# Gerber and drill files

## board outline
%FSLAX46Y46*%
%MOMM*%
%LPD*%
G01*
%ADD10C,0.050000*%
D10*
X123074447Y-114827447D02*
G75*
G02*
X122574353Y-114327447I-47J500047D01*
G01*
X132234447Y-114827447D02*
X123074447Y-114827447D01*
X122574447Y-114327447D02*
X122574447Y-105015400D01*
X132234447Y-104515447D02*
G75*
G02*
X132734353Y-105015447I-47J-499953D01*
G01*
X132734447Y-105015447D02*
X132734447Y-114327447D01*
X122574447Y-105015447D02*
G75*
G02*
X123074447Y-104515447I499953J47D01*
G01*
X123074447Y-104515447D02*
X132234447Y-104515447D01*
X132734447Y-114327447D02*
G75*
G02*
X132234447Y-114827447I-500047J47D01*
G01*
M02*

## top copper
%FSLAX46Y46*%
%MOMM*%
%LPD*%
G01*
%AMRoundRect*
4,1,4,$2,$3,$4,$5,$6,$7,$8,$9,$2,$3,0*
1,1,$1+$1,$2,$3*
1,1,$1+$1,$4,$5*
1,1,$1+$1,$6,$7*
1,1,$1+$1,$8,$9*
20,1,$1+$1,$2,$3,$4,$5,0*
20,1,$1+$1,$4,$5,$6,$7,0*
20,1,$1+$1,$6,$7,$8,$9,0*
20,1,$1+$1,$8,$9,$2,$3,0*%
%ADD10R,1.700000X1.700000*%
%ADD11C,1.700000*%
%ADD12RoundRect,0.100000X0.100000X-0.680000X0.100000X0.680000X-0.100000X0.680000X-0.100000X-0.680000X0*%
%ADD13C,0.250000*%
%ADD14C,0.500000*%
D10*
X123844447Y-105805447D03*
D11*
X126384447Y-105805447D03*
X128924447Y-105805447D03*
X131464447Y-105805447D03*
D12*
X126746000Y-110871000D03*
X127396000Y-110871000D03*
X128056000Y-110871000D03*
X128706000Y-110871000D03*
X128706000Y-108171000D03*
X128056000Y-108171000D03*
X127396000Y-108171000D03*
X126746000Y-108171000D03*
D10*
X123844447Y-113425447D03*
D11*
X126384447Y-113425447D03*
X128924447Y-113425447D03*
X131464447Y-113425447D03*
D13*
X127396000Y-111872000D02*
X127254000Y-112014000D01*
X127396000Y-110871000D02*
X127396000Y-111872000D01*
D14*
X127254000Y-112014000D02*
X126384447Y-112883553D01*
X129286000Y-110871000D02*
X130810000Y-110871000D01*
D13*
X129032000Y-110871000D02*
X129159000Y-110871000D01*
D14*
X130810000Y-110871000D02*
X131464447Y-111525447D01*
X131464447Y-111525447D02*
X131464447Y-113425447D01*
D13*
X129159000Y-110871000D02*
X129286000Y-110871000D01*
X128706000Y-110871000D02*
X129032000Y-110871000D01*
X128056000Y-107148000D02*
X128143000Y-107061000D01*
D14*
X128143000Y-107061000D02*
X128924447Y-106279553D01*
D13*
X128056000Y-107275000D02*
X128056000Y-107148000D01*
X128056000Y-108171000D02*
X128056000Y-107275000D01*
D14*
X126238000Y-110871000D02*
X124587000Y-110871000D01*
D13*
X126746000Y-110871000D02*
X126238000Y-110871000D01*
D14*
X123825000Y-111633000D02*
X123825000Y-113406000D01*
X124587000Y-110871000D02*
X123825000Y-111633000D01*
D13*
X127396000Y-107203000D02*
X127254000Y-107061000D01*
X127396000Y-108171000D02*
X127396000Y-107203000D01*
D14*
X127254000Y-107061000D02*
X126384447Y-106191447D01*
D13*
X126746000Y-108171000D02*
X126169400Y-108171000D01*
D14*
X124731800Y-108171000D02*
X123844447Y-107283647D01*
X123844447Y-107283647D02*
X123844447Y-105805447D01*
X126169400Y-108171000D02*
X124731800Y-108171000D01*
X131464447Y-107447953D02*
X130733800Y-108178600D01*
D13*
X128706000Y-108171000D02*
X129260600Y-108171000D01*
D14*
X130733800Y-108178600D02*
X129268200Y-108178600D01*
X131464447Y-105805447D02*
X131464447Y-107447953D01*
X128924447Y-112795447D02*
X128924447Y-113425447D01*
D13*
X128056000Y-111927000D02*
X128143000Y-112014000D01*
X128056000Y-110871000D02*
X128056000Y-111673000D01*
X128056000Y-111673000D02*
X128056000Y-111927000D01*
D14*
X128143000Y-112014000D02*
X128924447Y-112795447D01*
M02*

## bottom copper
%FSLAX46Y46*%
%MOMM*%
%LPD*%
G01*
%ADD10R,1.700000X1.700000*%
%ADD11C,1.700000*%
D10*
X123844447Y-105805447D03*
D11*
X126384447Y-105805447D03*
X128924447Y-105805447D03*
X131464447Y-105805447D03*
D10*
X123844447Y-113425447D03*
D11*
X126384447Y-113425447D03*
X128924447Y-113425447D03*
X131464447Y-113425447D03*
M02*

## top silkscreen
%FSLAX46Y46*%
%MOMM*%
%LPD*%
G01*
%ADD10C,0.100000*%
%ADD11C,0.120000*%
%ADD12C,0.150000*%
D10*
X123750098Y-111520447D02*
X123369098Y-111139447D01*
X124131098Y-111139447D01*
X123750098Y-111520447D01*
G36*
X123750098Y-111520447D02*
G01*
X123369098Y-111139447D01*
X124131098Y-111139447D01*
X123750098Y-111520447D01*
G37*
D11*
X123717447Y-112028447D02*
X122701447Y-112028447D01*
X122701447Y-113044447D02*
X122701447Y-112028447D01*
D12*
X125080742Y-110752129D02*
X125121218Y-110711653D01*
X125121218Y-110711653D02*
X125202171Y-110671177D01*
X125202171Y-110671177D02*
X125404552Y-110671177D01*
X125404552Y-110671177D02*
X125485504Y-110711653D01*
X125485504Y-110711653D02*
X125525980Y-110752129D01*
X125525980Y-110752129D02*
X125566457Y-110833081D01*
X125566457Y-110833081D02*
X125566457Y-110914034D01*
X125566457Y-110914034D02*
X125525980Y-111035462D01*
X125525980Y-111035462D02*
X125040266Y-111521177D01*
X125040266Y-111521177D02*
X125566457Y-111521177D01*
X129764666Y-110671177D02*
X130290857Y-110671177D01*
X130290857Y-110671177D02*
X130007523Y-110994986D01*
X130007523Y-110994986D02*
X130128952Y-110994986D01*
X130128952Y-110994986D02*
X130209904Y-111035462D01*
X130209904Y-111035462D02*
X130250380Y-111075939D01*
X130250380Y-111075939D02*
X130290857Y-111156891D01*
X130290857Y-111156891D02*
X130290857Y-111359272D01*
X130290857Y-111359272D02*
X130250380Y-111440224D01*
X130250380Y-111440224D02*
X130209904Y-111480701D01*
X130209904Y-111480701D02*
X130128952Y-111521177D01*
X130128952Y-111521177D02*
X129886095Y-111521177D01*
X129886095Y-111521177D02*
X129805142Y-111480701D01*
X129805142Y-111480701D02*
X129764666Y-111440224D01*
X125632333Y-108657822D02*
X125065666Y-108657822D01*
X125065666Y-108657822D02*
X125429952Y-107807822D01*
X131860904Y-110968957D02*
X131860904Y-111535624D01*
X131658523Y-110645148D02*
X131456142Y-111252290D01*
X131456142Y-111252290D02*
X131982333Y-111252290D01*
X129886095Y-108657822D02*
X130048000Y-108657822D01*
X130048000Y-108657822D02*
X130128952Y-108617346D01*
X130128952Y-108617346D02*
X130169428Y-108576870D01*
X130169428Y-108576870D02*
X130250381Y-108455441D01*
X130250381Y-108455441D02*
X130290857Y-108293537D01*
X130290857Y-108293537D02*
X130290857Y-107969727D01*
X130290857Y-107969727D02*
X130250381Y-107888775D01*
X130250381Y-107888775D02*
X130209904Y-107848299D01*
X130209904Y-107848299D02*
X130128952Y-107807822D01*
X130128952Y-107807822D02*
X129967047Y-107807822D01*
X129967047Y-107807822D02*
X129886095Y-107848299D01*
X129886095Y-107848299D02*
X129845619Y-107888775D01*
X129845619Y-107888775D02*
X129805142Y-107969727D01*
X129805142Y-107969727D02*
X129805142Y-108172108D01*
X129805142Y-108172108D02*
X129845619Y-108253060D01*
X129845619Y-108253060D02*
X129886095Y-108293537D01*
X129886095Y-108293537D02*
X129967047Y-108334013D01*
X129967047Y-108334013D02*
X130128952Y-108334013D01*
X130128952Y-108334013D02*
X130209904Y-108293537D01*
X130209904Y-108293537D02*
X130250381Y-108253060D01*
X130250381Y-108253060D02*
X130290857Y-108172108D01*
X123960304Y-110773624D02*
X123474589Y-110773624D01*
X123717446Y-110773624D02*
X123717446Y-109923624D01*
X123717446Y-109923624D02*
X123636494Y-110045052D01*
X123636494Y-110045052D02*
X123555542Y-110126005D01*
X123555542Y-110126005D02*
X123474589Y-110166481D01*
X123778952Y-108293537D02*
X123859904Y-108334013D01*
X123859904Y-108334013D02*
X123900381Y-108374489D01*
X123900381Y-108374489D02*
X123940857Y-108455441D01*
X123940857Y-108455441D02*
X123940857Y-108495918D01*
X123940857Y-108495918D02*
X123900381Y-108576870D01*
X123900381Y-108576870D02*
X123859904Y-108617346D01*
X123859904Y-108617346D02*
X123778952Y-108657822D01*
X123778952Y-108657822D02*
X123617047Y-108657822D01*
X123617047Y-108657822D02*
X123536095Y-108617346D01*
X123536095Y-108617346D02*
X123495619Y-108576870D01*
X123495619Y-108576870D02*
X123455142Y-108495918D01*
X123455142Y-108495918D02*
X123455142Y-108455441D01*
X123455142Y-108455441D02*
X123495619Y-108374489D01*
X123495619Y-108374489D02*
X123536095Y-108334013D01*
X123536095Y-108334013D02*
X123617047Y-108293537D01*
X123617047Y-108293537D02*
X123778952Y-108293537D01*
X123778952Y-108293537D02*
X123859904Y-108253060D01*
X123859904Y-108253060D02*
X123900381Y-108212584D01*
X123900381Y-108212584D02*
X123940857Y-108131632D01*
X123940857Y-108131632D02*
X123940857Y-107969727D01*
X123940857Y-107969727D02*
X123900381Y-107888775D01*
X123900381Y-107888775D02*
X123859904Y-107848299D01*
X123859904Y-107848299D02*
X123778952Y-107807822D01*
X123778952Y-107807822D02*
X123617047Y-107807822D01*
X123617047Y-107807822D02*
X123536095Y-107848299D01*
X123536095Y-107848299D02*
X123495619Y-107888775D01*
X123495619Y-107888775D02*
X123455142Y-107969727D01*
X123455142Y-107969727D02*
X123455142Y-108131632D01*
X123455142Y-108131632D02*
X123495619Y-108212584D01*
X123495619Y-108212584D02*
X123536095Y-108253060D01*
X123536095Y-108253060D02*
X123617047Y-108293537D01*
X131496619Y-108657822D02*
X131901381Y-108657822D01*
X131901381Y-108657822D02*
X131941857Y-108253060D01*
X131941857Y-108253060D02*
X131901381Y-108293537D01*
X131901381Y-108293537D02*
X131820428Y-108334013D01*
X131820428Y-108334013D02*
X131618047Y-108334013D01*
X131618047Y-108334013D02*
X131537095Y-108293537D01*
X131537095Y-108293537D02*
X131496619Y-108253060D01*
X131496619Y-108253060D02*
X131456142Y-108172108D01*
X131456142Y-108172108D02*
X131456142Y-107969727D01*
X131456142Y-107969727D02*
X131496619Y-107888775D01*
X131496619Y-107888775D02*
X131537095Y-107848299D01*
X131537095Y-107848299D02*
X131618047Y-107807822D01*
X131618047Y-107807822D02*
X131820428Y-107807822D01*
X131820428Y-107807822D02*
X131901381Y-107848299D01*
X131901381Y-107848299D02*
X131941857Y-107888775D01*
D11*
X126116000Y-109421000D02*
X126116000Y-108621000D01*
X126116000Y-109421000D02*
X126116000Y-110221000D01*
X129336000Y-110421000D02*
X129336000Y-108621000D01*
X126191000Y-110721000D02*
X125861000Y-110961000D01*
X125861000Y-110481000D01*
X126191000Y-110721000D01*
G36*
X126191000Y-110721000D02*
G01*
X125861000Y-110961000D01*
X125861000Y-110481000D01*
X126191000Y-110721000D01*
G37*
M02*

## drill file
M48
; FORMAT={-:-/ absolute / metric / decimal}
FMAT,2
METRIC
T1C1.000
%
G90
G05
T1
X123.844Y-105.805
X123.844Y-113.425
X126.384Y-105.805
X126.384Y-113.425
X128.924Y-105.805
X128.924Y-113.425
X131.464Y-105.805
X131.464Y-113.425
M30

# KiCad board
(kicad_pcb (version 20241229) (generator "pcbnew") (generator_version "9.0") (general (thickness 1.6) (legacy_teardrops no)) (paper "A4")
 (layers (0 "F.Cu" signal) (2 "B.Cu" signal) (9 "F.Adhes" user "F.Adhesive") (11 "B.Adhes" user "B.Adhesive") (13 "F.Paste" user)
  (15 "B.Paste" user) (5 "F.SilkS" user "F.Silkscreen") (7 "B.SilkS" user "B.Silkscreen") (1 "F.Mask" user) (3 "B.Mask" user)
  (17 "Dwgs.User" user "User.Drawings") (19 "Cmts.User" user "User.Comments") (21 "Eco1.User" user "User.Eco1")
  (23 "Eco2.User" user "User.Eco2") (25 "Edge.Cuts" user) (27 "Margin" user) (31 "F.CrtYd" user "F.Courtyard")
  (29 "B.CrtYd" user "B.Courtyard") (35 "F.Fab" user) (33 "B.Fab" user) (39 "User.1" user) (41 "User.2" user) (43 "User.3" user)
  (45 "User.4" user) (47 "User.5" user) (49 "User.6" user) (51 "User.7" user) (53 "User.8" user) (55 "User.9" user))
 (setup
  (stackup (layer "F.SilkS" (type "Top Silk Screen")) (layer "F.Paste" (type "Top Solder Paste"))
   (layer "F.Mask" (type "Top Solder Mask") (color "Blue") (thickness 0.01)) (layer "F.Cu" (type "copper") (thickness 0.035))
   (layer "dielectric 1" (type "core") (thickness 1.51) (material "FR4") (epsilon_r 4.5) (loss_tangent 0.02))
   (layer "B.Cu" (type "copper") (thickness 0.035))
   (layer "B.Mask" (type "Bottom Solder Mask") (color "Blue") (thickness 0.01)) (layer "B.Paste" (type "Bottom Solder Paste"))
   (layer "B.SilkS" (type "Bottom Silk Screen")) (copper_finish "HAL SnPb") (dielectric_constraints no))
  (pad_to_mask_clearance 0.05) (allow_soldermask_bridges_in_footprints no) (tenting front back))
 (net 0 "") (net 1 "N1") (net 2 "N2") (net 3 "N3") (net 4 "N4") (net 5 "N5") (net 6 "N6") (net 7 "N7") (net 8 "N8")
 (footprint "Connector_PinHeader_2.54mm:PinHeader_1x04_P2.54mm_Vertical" (layer "F.Cu") (at 123.844447 105.805447 90)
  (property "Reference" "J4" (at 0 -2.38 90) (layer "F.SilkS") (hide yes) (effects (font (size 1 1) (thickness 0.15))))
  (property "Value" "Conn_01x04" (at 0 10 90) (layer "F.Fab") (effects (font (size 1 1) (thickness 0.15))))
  (pad "1" thru_hole rect (at 0 0 90) (size 1.7 1.7) (drill 1) (layers "*.Cu" "*.Mask") (remove_unused_layers no) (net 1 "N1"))
  (pad "2" thru_hole circle (at 0 2.54 90) (size 1.7 1.7) (drill 1) (layers "*.Cu" "*.Mask") (remove_unused_layers no) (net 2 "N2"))
  (pad "3" thru_hole circle (at 0 5.08 90) (size 1.7 1.7) (drill 1) (layers "*.Cu" "*.Mask") (remove_unused_layers no) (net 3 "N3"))
  (pad "4" thru_hole circle (at 0 7.62 90) (size 1.7 1.7) (drill 1) (layers "*.Cu" "*.Mask") (remove_unused_layers no) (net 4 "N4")))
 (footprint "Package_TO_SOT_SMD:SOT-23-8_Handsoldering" (layer "F.Cu") (at 127.726 109.521 90)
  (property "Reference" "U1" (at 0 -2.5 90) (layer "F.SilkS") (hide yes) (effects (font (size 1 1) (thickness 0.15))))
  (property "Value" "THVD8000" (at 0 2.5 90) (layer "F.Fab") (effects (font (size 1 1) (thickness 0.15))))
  (fp_line (start 0.1 -1.61) (end 0.9 -1.61) (stroke (width 0.12) (type solid)) (layer "F.SilkS"))
  (fp_line (start 0.1 -1.61) (end -0.7 -1.61) (stroke (width 0.12) (type solid)) (layer "F.SilkS"))
  (fp_line (start -0.9 1.61) (end 0.9 1.61) (stroke (width 0.12) (type solid)) (layer "F.SilkS"))
  (fp_poly
   (pts (xy -1.2 -1.535) (xy -1.44 -1.865) (xy -0.96 -1.865) (xy -1.2 -1.535)) (stroke (width 0.12) (type solid)) (fill yes)
   (layer "F.SilkS"))
  (pad "1" smd roundrect (at -1.35 -0.98 90) (size 1.56 0.4) (layers "F.Cu" "F.Mask" "F.Paste") (roundrect_rratio 0.25) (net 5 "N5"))
  (pad "2" smd roundrect (at -1.35 -0.33 90) (size 1.56 0.4) (layers "F.Cu" "F.Mask" "F.Paste") (roundrect_rratio 0.25) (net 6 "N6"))
  (pad "3" smd roundrect (at -1.35 0.33 90) (size 1.56 0.4) (layers "F.Cu" "F.Mask" "F.Paste") (roundrect_rratio 0.25) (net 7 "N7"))
  (pad "4" smd roundrect (at -1.35 0.98 90) (size 1.56 0.4) (layers "F.Cu" "F.Mask" "F.Paste") (roundrect_rratio 0.25) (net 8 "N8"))
  (pad "5" smd roundrect (at 1.35 0.98 90) (size 1.56 0.4) (layers "F.Cu" "F.Mask" "F.Paste") (roundrect_rratio 0.25) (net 4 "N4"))
  (pad "6" smd roundrect (at 1.35 0.33 90) (size 1.56 0.4) (layers "F.Cu" "F.Mask" "F.Paste") (roundrect_rratio 0.25) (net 3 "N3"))
  (pad "7" smd roundrect (at 1.35 -0.33 90) (size 1.56 0.4) (layers "F.Cu" "F.Mask" "F.Paste") (roundrect_rratio 0.25) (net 2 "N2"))
  (pad "8" smd roundrect (at 1.35 -0.98 90) (size 1.56 0.4) (layers "F.Cu" "F.Mask" "F.Paste") (roundrect_rratio 0.25) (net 1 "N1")))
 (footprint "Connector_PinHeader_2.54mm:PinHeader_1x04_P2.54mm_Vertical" (layer "F.Cu") (at 123.844447 113.425447 90)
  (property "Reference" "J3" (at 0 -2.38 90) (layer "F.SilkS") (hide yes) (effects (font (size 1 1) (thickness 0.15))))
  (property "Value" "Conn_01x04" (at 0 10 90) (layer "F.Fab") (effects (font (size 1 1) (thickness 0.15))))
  (pad "1" thru_hole rect (at 0 0 90) (size 1.7 1.7) (drill 1) (layers "*.Cu" "*.Mask") (remove_unused_layers no) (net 5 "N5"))
  (pad "2" thru_hole circle (at 0 2.54 90) (size 1.7 1.7) (drill 1) (layers "*.Cu" "*.Mask") (remove_unused_layers no) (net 6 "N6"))
  (pad "3" thru_hole circle (at 0 5.08 90) (size 1.7 1.7) (drill 1) (layers "*.Cu" "*.Mask") (remove_unused_layers no) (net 7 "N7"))
  (pad "4" thru_hole circle (at 0 7.62 90) (size 1.7 1.7) (drill 1) (layers "*.Cu" "*.Mask") (remove_unused_layers no) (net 8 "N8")))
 (gr_poly
  (pts (xy 123.750098 111.520447) (xy 123.369098 111.139447) (xy 124.131098 111.139447)) (stroke (width 0.1) (type solid)) (fill yes)
  (layer "F.SilkS"))
 (gr_line (start 123.717447 112.028447) (end 122.701447 112.028447) (stroke (width 0.12) (type default)) (layer "F.SilkS"))
 (gr_line (start 122.701447 113.044447) (end 122.701447 112.028447) (stroke (width 0.12) (type default)) (layer "F.SilkS"))
 (gr_arc (start 123.074447 114.827447) (mid 122.720894 114.681) (end 122.574447 114.327447) (stroke (width 0.05) (type default))
  (locked yes) (layer "Edge.Cuts"))
 (gr_line (start 132.234447 114.827447) (end 123.074447 114.827447) (stroke (width 0.05) (type default)) (locked yes) (layer "Edge.Cuts"))
 (gr_line (start 122.574447 114.327447) (end 122.574447 105.0154) (stroke (width 0.05) (type default)) (locked yes) (layer "Edge.Cuts"))
 (gr_arc (start 132.234447 104.515447) (mid 132.588 104.661894) (end 132.734447 105.015447) (stroke (width 0.05) (type default))
  (locked yes) (layer "Edge.Cuts"))
 (gr_line (start 132.734447 105.015447) (end 132.734447 114.327447) (stroke (width 0.05) (type default)) (locked yes) (layer "Edge.Cuts"))
 (gr_arc (start 122.574447 105.015447) (mid 122.720894 104.661894) (end 123.074447 104.515447) (stroke (width 0.05) (type default))
  (locked yes) (layer "Edge.Cuts"))
 (gr_line (start 123.074447 104.515447) (end 132.234447 104.515447) (stroke (width 0.05) (type default)) (locked yes) (layer "Edge.Cuts"))
 (gr_arc (start 132.734447 114.327447) (mid 132.588 114.681) (end 132.234447 114.827447) (stroke (width 0.05) (type default)) (locked yes)
  (layer "Edge.Cuts"))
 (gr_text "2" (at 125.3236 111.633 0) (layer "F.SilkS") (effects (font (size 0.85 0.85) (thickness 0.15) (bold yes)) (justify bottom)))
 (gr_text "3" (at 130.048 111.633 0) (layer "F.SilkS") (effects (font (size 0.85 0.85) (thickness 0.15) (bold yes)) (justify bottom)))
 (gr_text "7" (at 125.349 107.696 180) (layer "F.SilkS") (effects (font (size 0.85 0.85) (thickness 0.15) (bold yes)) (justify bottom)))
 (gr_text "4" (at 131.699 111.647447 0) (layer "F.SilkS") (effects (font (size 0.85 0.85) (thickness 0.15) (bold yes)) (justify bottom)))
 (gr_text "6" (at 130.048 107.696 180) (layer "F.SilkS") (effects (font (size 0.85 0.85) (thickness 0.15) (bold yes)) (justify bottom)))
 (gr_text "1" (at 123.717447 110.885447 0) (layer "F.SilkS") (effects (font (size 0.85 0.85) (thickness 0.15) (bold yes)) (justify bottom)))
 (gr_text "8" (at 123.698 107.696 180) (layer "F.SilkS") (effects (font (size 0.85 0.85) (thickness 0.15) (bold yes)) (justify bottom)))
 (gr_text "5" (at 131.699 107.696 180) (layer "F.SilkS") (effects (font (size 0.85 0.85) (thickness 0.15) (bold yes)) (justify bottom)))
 (segment (start 127.396 111.872) (end 127.254 112.014) (width 0.25) (layer "F.Cu") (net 6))
 (segment (start 127.396 110.871) (end 127.396 111.872) (width 0.25) (layer "F.Cu") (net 6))
 (segment (start 127.254 112.014) (end 126.384447 112.883553) (width 0.5) (layer "F.Cu") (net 6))
 (segment (start 129.286 110.871) (end 130.81 110.871) (width 0.5) (layer "F.Cu") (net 8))
 (segment (start 129.032 110.871) (end 129.159 110.871) (width 0.25) (layer "F.Cu") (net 8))
 (segment (start 130.81 110.871) (end 131.464447 111.525447) (width 0.5) (layer "F.Cu") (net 8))
 (segment (start 131.464447 111.525447) (end 131.464447 113.425447) (width 0.5) (layer "F.Cu") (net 8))
 (segment (start 129.159 110.871) (end 129.286 110.871) (width 0.25) (layer "F.Cu") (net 8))
 (segment (start 128.706 110.871) (end 129.032 110.871) (width 0.25) (layer "F.Cu") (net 8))
 (segment (start 128.056 107.148) (end 128.143 107.061) (width 0.25) (layer "F.Cu") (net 3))
 (segment (start 128.143 107.061) (end 128.924447 106.279553) (width 0.5) (layer "F.Cu") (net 3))
 (segment (start 128.056 107.275) (end 128.056 107.148) (width 0.25) (layer "F.Cu") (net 3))
 (segment (start 128.056 108.171) (end 128.056 107.275) (width 0.25) (layer "F.Cu") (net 3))
 (segment (start 126.238 110.871) (end 124.587 110.871) (width 0.5) (layer "F.Cu") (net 5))
 (segment (start 126.746 110.871) (end 126.238 110.871) (width 0.25) (layer "F.Cu") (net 5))
 (segment (start 123.825 111.633) (end 123.825 113.406) (width 0.5) (layer "F.Cu") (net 5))
 (segment (start 124.587 110.871) (end 123.825 111.633) (width 0.5) (layer "F.Cu") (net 5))
 (segment (start 127.396 107.203) (end 127.254 107.061) (width 0.25) (layer "F.Cu") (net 2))
 (segment (start 127.396 108.171) (end 127.396 107.203) (width 0.25) (layer "F.Cu") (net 2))
 (segment (start 127.254 107.061) (end 126.384447 106.191447) (width 0.5) (layer "F.Cu") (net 2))
 (segment (start 126.746 108.171) (end 126.1694 108.171) (width 0.25) (layer "F.Cu") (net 1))
 (segment (start 124.7318 108.171) (end 123.844447 107.283647) (width 0.5) (layer "F.Cu") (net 1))
 (segment (start 123.844447 107.283647) (end 123.844447 105.805447) (width 0.5) (layer "F.Cu") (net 1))
 (segment (start 126.1694 108.171) (end 124.7318 108.171) (width 0.5) (layer "F.Cu") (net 1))
 (segment (start 131.464447 107.447953) (end 130.7338 108.1786) (width 0.5) (layer "F.Cu") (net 4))
 (segment (start 128.706 108.171) (end 129.2606 108.171) (width 0.25) (layer "F.Cu") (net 4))
 (segment (start 130.7338 108.1786) (end 129.2682 108.1786) (width 0.5) (layer "F.Cu") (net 4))
 (segment (start 131.464447 105.805447) (end 131.464447 107.447953) (width 0.5) (layer "F.Cu") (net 4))
 (segment (start 128.924447 112.795447) (end 128.924447 113.425447) (width 0.5) (layer "F.Cu") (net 7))
 (segment (start 128.056 111.927) (end 128.143 112.014) (width 0.25) (layer "F.Cu") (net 7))
 (segment (start 128.056 110.871) (end 128.056 111.673) (width 0.25) (layer "F.Cu") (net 7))
 (segment (start 128.056 111.673) (end 128.056 111.927) (width 0.25) (layer "F.Cu") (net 7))
 (segment (start 128.143 112.014) (end 128.924447 112.795447) (width 0.5) (layer "F.Cu") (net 7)))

